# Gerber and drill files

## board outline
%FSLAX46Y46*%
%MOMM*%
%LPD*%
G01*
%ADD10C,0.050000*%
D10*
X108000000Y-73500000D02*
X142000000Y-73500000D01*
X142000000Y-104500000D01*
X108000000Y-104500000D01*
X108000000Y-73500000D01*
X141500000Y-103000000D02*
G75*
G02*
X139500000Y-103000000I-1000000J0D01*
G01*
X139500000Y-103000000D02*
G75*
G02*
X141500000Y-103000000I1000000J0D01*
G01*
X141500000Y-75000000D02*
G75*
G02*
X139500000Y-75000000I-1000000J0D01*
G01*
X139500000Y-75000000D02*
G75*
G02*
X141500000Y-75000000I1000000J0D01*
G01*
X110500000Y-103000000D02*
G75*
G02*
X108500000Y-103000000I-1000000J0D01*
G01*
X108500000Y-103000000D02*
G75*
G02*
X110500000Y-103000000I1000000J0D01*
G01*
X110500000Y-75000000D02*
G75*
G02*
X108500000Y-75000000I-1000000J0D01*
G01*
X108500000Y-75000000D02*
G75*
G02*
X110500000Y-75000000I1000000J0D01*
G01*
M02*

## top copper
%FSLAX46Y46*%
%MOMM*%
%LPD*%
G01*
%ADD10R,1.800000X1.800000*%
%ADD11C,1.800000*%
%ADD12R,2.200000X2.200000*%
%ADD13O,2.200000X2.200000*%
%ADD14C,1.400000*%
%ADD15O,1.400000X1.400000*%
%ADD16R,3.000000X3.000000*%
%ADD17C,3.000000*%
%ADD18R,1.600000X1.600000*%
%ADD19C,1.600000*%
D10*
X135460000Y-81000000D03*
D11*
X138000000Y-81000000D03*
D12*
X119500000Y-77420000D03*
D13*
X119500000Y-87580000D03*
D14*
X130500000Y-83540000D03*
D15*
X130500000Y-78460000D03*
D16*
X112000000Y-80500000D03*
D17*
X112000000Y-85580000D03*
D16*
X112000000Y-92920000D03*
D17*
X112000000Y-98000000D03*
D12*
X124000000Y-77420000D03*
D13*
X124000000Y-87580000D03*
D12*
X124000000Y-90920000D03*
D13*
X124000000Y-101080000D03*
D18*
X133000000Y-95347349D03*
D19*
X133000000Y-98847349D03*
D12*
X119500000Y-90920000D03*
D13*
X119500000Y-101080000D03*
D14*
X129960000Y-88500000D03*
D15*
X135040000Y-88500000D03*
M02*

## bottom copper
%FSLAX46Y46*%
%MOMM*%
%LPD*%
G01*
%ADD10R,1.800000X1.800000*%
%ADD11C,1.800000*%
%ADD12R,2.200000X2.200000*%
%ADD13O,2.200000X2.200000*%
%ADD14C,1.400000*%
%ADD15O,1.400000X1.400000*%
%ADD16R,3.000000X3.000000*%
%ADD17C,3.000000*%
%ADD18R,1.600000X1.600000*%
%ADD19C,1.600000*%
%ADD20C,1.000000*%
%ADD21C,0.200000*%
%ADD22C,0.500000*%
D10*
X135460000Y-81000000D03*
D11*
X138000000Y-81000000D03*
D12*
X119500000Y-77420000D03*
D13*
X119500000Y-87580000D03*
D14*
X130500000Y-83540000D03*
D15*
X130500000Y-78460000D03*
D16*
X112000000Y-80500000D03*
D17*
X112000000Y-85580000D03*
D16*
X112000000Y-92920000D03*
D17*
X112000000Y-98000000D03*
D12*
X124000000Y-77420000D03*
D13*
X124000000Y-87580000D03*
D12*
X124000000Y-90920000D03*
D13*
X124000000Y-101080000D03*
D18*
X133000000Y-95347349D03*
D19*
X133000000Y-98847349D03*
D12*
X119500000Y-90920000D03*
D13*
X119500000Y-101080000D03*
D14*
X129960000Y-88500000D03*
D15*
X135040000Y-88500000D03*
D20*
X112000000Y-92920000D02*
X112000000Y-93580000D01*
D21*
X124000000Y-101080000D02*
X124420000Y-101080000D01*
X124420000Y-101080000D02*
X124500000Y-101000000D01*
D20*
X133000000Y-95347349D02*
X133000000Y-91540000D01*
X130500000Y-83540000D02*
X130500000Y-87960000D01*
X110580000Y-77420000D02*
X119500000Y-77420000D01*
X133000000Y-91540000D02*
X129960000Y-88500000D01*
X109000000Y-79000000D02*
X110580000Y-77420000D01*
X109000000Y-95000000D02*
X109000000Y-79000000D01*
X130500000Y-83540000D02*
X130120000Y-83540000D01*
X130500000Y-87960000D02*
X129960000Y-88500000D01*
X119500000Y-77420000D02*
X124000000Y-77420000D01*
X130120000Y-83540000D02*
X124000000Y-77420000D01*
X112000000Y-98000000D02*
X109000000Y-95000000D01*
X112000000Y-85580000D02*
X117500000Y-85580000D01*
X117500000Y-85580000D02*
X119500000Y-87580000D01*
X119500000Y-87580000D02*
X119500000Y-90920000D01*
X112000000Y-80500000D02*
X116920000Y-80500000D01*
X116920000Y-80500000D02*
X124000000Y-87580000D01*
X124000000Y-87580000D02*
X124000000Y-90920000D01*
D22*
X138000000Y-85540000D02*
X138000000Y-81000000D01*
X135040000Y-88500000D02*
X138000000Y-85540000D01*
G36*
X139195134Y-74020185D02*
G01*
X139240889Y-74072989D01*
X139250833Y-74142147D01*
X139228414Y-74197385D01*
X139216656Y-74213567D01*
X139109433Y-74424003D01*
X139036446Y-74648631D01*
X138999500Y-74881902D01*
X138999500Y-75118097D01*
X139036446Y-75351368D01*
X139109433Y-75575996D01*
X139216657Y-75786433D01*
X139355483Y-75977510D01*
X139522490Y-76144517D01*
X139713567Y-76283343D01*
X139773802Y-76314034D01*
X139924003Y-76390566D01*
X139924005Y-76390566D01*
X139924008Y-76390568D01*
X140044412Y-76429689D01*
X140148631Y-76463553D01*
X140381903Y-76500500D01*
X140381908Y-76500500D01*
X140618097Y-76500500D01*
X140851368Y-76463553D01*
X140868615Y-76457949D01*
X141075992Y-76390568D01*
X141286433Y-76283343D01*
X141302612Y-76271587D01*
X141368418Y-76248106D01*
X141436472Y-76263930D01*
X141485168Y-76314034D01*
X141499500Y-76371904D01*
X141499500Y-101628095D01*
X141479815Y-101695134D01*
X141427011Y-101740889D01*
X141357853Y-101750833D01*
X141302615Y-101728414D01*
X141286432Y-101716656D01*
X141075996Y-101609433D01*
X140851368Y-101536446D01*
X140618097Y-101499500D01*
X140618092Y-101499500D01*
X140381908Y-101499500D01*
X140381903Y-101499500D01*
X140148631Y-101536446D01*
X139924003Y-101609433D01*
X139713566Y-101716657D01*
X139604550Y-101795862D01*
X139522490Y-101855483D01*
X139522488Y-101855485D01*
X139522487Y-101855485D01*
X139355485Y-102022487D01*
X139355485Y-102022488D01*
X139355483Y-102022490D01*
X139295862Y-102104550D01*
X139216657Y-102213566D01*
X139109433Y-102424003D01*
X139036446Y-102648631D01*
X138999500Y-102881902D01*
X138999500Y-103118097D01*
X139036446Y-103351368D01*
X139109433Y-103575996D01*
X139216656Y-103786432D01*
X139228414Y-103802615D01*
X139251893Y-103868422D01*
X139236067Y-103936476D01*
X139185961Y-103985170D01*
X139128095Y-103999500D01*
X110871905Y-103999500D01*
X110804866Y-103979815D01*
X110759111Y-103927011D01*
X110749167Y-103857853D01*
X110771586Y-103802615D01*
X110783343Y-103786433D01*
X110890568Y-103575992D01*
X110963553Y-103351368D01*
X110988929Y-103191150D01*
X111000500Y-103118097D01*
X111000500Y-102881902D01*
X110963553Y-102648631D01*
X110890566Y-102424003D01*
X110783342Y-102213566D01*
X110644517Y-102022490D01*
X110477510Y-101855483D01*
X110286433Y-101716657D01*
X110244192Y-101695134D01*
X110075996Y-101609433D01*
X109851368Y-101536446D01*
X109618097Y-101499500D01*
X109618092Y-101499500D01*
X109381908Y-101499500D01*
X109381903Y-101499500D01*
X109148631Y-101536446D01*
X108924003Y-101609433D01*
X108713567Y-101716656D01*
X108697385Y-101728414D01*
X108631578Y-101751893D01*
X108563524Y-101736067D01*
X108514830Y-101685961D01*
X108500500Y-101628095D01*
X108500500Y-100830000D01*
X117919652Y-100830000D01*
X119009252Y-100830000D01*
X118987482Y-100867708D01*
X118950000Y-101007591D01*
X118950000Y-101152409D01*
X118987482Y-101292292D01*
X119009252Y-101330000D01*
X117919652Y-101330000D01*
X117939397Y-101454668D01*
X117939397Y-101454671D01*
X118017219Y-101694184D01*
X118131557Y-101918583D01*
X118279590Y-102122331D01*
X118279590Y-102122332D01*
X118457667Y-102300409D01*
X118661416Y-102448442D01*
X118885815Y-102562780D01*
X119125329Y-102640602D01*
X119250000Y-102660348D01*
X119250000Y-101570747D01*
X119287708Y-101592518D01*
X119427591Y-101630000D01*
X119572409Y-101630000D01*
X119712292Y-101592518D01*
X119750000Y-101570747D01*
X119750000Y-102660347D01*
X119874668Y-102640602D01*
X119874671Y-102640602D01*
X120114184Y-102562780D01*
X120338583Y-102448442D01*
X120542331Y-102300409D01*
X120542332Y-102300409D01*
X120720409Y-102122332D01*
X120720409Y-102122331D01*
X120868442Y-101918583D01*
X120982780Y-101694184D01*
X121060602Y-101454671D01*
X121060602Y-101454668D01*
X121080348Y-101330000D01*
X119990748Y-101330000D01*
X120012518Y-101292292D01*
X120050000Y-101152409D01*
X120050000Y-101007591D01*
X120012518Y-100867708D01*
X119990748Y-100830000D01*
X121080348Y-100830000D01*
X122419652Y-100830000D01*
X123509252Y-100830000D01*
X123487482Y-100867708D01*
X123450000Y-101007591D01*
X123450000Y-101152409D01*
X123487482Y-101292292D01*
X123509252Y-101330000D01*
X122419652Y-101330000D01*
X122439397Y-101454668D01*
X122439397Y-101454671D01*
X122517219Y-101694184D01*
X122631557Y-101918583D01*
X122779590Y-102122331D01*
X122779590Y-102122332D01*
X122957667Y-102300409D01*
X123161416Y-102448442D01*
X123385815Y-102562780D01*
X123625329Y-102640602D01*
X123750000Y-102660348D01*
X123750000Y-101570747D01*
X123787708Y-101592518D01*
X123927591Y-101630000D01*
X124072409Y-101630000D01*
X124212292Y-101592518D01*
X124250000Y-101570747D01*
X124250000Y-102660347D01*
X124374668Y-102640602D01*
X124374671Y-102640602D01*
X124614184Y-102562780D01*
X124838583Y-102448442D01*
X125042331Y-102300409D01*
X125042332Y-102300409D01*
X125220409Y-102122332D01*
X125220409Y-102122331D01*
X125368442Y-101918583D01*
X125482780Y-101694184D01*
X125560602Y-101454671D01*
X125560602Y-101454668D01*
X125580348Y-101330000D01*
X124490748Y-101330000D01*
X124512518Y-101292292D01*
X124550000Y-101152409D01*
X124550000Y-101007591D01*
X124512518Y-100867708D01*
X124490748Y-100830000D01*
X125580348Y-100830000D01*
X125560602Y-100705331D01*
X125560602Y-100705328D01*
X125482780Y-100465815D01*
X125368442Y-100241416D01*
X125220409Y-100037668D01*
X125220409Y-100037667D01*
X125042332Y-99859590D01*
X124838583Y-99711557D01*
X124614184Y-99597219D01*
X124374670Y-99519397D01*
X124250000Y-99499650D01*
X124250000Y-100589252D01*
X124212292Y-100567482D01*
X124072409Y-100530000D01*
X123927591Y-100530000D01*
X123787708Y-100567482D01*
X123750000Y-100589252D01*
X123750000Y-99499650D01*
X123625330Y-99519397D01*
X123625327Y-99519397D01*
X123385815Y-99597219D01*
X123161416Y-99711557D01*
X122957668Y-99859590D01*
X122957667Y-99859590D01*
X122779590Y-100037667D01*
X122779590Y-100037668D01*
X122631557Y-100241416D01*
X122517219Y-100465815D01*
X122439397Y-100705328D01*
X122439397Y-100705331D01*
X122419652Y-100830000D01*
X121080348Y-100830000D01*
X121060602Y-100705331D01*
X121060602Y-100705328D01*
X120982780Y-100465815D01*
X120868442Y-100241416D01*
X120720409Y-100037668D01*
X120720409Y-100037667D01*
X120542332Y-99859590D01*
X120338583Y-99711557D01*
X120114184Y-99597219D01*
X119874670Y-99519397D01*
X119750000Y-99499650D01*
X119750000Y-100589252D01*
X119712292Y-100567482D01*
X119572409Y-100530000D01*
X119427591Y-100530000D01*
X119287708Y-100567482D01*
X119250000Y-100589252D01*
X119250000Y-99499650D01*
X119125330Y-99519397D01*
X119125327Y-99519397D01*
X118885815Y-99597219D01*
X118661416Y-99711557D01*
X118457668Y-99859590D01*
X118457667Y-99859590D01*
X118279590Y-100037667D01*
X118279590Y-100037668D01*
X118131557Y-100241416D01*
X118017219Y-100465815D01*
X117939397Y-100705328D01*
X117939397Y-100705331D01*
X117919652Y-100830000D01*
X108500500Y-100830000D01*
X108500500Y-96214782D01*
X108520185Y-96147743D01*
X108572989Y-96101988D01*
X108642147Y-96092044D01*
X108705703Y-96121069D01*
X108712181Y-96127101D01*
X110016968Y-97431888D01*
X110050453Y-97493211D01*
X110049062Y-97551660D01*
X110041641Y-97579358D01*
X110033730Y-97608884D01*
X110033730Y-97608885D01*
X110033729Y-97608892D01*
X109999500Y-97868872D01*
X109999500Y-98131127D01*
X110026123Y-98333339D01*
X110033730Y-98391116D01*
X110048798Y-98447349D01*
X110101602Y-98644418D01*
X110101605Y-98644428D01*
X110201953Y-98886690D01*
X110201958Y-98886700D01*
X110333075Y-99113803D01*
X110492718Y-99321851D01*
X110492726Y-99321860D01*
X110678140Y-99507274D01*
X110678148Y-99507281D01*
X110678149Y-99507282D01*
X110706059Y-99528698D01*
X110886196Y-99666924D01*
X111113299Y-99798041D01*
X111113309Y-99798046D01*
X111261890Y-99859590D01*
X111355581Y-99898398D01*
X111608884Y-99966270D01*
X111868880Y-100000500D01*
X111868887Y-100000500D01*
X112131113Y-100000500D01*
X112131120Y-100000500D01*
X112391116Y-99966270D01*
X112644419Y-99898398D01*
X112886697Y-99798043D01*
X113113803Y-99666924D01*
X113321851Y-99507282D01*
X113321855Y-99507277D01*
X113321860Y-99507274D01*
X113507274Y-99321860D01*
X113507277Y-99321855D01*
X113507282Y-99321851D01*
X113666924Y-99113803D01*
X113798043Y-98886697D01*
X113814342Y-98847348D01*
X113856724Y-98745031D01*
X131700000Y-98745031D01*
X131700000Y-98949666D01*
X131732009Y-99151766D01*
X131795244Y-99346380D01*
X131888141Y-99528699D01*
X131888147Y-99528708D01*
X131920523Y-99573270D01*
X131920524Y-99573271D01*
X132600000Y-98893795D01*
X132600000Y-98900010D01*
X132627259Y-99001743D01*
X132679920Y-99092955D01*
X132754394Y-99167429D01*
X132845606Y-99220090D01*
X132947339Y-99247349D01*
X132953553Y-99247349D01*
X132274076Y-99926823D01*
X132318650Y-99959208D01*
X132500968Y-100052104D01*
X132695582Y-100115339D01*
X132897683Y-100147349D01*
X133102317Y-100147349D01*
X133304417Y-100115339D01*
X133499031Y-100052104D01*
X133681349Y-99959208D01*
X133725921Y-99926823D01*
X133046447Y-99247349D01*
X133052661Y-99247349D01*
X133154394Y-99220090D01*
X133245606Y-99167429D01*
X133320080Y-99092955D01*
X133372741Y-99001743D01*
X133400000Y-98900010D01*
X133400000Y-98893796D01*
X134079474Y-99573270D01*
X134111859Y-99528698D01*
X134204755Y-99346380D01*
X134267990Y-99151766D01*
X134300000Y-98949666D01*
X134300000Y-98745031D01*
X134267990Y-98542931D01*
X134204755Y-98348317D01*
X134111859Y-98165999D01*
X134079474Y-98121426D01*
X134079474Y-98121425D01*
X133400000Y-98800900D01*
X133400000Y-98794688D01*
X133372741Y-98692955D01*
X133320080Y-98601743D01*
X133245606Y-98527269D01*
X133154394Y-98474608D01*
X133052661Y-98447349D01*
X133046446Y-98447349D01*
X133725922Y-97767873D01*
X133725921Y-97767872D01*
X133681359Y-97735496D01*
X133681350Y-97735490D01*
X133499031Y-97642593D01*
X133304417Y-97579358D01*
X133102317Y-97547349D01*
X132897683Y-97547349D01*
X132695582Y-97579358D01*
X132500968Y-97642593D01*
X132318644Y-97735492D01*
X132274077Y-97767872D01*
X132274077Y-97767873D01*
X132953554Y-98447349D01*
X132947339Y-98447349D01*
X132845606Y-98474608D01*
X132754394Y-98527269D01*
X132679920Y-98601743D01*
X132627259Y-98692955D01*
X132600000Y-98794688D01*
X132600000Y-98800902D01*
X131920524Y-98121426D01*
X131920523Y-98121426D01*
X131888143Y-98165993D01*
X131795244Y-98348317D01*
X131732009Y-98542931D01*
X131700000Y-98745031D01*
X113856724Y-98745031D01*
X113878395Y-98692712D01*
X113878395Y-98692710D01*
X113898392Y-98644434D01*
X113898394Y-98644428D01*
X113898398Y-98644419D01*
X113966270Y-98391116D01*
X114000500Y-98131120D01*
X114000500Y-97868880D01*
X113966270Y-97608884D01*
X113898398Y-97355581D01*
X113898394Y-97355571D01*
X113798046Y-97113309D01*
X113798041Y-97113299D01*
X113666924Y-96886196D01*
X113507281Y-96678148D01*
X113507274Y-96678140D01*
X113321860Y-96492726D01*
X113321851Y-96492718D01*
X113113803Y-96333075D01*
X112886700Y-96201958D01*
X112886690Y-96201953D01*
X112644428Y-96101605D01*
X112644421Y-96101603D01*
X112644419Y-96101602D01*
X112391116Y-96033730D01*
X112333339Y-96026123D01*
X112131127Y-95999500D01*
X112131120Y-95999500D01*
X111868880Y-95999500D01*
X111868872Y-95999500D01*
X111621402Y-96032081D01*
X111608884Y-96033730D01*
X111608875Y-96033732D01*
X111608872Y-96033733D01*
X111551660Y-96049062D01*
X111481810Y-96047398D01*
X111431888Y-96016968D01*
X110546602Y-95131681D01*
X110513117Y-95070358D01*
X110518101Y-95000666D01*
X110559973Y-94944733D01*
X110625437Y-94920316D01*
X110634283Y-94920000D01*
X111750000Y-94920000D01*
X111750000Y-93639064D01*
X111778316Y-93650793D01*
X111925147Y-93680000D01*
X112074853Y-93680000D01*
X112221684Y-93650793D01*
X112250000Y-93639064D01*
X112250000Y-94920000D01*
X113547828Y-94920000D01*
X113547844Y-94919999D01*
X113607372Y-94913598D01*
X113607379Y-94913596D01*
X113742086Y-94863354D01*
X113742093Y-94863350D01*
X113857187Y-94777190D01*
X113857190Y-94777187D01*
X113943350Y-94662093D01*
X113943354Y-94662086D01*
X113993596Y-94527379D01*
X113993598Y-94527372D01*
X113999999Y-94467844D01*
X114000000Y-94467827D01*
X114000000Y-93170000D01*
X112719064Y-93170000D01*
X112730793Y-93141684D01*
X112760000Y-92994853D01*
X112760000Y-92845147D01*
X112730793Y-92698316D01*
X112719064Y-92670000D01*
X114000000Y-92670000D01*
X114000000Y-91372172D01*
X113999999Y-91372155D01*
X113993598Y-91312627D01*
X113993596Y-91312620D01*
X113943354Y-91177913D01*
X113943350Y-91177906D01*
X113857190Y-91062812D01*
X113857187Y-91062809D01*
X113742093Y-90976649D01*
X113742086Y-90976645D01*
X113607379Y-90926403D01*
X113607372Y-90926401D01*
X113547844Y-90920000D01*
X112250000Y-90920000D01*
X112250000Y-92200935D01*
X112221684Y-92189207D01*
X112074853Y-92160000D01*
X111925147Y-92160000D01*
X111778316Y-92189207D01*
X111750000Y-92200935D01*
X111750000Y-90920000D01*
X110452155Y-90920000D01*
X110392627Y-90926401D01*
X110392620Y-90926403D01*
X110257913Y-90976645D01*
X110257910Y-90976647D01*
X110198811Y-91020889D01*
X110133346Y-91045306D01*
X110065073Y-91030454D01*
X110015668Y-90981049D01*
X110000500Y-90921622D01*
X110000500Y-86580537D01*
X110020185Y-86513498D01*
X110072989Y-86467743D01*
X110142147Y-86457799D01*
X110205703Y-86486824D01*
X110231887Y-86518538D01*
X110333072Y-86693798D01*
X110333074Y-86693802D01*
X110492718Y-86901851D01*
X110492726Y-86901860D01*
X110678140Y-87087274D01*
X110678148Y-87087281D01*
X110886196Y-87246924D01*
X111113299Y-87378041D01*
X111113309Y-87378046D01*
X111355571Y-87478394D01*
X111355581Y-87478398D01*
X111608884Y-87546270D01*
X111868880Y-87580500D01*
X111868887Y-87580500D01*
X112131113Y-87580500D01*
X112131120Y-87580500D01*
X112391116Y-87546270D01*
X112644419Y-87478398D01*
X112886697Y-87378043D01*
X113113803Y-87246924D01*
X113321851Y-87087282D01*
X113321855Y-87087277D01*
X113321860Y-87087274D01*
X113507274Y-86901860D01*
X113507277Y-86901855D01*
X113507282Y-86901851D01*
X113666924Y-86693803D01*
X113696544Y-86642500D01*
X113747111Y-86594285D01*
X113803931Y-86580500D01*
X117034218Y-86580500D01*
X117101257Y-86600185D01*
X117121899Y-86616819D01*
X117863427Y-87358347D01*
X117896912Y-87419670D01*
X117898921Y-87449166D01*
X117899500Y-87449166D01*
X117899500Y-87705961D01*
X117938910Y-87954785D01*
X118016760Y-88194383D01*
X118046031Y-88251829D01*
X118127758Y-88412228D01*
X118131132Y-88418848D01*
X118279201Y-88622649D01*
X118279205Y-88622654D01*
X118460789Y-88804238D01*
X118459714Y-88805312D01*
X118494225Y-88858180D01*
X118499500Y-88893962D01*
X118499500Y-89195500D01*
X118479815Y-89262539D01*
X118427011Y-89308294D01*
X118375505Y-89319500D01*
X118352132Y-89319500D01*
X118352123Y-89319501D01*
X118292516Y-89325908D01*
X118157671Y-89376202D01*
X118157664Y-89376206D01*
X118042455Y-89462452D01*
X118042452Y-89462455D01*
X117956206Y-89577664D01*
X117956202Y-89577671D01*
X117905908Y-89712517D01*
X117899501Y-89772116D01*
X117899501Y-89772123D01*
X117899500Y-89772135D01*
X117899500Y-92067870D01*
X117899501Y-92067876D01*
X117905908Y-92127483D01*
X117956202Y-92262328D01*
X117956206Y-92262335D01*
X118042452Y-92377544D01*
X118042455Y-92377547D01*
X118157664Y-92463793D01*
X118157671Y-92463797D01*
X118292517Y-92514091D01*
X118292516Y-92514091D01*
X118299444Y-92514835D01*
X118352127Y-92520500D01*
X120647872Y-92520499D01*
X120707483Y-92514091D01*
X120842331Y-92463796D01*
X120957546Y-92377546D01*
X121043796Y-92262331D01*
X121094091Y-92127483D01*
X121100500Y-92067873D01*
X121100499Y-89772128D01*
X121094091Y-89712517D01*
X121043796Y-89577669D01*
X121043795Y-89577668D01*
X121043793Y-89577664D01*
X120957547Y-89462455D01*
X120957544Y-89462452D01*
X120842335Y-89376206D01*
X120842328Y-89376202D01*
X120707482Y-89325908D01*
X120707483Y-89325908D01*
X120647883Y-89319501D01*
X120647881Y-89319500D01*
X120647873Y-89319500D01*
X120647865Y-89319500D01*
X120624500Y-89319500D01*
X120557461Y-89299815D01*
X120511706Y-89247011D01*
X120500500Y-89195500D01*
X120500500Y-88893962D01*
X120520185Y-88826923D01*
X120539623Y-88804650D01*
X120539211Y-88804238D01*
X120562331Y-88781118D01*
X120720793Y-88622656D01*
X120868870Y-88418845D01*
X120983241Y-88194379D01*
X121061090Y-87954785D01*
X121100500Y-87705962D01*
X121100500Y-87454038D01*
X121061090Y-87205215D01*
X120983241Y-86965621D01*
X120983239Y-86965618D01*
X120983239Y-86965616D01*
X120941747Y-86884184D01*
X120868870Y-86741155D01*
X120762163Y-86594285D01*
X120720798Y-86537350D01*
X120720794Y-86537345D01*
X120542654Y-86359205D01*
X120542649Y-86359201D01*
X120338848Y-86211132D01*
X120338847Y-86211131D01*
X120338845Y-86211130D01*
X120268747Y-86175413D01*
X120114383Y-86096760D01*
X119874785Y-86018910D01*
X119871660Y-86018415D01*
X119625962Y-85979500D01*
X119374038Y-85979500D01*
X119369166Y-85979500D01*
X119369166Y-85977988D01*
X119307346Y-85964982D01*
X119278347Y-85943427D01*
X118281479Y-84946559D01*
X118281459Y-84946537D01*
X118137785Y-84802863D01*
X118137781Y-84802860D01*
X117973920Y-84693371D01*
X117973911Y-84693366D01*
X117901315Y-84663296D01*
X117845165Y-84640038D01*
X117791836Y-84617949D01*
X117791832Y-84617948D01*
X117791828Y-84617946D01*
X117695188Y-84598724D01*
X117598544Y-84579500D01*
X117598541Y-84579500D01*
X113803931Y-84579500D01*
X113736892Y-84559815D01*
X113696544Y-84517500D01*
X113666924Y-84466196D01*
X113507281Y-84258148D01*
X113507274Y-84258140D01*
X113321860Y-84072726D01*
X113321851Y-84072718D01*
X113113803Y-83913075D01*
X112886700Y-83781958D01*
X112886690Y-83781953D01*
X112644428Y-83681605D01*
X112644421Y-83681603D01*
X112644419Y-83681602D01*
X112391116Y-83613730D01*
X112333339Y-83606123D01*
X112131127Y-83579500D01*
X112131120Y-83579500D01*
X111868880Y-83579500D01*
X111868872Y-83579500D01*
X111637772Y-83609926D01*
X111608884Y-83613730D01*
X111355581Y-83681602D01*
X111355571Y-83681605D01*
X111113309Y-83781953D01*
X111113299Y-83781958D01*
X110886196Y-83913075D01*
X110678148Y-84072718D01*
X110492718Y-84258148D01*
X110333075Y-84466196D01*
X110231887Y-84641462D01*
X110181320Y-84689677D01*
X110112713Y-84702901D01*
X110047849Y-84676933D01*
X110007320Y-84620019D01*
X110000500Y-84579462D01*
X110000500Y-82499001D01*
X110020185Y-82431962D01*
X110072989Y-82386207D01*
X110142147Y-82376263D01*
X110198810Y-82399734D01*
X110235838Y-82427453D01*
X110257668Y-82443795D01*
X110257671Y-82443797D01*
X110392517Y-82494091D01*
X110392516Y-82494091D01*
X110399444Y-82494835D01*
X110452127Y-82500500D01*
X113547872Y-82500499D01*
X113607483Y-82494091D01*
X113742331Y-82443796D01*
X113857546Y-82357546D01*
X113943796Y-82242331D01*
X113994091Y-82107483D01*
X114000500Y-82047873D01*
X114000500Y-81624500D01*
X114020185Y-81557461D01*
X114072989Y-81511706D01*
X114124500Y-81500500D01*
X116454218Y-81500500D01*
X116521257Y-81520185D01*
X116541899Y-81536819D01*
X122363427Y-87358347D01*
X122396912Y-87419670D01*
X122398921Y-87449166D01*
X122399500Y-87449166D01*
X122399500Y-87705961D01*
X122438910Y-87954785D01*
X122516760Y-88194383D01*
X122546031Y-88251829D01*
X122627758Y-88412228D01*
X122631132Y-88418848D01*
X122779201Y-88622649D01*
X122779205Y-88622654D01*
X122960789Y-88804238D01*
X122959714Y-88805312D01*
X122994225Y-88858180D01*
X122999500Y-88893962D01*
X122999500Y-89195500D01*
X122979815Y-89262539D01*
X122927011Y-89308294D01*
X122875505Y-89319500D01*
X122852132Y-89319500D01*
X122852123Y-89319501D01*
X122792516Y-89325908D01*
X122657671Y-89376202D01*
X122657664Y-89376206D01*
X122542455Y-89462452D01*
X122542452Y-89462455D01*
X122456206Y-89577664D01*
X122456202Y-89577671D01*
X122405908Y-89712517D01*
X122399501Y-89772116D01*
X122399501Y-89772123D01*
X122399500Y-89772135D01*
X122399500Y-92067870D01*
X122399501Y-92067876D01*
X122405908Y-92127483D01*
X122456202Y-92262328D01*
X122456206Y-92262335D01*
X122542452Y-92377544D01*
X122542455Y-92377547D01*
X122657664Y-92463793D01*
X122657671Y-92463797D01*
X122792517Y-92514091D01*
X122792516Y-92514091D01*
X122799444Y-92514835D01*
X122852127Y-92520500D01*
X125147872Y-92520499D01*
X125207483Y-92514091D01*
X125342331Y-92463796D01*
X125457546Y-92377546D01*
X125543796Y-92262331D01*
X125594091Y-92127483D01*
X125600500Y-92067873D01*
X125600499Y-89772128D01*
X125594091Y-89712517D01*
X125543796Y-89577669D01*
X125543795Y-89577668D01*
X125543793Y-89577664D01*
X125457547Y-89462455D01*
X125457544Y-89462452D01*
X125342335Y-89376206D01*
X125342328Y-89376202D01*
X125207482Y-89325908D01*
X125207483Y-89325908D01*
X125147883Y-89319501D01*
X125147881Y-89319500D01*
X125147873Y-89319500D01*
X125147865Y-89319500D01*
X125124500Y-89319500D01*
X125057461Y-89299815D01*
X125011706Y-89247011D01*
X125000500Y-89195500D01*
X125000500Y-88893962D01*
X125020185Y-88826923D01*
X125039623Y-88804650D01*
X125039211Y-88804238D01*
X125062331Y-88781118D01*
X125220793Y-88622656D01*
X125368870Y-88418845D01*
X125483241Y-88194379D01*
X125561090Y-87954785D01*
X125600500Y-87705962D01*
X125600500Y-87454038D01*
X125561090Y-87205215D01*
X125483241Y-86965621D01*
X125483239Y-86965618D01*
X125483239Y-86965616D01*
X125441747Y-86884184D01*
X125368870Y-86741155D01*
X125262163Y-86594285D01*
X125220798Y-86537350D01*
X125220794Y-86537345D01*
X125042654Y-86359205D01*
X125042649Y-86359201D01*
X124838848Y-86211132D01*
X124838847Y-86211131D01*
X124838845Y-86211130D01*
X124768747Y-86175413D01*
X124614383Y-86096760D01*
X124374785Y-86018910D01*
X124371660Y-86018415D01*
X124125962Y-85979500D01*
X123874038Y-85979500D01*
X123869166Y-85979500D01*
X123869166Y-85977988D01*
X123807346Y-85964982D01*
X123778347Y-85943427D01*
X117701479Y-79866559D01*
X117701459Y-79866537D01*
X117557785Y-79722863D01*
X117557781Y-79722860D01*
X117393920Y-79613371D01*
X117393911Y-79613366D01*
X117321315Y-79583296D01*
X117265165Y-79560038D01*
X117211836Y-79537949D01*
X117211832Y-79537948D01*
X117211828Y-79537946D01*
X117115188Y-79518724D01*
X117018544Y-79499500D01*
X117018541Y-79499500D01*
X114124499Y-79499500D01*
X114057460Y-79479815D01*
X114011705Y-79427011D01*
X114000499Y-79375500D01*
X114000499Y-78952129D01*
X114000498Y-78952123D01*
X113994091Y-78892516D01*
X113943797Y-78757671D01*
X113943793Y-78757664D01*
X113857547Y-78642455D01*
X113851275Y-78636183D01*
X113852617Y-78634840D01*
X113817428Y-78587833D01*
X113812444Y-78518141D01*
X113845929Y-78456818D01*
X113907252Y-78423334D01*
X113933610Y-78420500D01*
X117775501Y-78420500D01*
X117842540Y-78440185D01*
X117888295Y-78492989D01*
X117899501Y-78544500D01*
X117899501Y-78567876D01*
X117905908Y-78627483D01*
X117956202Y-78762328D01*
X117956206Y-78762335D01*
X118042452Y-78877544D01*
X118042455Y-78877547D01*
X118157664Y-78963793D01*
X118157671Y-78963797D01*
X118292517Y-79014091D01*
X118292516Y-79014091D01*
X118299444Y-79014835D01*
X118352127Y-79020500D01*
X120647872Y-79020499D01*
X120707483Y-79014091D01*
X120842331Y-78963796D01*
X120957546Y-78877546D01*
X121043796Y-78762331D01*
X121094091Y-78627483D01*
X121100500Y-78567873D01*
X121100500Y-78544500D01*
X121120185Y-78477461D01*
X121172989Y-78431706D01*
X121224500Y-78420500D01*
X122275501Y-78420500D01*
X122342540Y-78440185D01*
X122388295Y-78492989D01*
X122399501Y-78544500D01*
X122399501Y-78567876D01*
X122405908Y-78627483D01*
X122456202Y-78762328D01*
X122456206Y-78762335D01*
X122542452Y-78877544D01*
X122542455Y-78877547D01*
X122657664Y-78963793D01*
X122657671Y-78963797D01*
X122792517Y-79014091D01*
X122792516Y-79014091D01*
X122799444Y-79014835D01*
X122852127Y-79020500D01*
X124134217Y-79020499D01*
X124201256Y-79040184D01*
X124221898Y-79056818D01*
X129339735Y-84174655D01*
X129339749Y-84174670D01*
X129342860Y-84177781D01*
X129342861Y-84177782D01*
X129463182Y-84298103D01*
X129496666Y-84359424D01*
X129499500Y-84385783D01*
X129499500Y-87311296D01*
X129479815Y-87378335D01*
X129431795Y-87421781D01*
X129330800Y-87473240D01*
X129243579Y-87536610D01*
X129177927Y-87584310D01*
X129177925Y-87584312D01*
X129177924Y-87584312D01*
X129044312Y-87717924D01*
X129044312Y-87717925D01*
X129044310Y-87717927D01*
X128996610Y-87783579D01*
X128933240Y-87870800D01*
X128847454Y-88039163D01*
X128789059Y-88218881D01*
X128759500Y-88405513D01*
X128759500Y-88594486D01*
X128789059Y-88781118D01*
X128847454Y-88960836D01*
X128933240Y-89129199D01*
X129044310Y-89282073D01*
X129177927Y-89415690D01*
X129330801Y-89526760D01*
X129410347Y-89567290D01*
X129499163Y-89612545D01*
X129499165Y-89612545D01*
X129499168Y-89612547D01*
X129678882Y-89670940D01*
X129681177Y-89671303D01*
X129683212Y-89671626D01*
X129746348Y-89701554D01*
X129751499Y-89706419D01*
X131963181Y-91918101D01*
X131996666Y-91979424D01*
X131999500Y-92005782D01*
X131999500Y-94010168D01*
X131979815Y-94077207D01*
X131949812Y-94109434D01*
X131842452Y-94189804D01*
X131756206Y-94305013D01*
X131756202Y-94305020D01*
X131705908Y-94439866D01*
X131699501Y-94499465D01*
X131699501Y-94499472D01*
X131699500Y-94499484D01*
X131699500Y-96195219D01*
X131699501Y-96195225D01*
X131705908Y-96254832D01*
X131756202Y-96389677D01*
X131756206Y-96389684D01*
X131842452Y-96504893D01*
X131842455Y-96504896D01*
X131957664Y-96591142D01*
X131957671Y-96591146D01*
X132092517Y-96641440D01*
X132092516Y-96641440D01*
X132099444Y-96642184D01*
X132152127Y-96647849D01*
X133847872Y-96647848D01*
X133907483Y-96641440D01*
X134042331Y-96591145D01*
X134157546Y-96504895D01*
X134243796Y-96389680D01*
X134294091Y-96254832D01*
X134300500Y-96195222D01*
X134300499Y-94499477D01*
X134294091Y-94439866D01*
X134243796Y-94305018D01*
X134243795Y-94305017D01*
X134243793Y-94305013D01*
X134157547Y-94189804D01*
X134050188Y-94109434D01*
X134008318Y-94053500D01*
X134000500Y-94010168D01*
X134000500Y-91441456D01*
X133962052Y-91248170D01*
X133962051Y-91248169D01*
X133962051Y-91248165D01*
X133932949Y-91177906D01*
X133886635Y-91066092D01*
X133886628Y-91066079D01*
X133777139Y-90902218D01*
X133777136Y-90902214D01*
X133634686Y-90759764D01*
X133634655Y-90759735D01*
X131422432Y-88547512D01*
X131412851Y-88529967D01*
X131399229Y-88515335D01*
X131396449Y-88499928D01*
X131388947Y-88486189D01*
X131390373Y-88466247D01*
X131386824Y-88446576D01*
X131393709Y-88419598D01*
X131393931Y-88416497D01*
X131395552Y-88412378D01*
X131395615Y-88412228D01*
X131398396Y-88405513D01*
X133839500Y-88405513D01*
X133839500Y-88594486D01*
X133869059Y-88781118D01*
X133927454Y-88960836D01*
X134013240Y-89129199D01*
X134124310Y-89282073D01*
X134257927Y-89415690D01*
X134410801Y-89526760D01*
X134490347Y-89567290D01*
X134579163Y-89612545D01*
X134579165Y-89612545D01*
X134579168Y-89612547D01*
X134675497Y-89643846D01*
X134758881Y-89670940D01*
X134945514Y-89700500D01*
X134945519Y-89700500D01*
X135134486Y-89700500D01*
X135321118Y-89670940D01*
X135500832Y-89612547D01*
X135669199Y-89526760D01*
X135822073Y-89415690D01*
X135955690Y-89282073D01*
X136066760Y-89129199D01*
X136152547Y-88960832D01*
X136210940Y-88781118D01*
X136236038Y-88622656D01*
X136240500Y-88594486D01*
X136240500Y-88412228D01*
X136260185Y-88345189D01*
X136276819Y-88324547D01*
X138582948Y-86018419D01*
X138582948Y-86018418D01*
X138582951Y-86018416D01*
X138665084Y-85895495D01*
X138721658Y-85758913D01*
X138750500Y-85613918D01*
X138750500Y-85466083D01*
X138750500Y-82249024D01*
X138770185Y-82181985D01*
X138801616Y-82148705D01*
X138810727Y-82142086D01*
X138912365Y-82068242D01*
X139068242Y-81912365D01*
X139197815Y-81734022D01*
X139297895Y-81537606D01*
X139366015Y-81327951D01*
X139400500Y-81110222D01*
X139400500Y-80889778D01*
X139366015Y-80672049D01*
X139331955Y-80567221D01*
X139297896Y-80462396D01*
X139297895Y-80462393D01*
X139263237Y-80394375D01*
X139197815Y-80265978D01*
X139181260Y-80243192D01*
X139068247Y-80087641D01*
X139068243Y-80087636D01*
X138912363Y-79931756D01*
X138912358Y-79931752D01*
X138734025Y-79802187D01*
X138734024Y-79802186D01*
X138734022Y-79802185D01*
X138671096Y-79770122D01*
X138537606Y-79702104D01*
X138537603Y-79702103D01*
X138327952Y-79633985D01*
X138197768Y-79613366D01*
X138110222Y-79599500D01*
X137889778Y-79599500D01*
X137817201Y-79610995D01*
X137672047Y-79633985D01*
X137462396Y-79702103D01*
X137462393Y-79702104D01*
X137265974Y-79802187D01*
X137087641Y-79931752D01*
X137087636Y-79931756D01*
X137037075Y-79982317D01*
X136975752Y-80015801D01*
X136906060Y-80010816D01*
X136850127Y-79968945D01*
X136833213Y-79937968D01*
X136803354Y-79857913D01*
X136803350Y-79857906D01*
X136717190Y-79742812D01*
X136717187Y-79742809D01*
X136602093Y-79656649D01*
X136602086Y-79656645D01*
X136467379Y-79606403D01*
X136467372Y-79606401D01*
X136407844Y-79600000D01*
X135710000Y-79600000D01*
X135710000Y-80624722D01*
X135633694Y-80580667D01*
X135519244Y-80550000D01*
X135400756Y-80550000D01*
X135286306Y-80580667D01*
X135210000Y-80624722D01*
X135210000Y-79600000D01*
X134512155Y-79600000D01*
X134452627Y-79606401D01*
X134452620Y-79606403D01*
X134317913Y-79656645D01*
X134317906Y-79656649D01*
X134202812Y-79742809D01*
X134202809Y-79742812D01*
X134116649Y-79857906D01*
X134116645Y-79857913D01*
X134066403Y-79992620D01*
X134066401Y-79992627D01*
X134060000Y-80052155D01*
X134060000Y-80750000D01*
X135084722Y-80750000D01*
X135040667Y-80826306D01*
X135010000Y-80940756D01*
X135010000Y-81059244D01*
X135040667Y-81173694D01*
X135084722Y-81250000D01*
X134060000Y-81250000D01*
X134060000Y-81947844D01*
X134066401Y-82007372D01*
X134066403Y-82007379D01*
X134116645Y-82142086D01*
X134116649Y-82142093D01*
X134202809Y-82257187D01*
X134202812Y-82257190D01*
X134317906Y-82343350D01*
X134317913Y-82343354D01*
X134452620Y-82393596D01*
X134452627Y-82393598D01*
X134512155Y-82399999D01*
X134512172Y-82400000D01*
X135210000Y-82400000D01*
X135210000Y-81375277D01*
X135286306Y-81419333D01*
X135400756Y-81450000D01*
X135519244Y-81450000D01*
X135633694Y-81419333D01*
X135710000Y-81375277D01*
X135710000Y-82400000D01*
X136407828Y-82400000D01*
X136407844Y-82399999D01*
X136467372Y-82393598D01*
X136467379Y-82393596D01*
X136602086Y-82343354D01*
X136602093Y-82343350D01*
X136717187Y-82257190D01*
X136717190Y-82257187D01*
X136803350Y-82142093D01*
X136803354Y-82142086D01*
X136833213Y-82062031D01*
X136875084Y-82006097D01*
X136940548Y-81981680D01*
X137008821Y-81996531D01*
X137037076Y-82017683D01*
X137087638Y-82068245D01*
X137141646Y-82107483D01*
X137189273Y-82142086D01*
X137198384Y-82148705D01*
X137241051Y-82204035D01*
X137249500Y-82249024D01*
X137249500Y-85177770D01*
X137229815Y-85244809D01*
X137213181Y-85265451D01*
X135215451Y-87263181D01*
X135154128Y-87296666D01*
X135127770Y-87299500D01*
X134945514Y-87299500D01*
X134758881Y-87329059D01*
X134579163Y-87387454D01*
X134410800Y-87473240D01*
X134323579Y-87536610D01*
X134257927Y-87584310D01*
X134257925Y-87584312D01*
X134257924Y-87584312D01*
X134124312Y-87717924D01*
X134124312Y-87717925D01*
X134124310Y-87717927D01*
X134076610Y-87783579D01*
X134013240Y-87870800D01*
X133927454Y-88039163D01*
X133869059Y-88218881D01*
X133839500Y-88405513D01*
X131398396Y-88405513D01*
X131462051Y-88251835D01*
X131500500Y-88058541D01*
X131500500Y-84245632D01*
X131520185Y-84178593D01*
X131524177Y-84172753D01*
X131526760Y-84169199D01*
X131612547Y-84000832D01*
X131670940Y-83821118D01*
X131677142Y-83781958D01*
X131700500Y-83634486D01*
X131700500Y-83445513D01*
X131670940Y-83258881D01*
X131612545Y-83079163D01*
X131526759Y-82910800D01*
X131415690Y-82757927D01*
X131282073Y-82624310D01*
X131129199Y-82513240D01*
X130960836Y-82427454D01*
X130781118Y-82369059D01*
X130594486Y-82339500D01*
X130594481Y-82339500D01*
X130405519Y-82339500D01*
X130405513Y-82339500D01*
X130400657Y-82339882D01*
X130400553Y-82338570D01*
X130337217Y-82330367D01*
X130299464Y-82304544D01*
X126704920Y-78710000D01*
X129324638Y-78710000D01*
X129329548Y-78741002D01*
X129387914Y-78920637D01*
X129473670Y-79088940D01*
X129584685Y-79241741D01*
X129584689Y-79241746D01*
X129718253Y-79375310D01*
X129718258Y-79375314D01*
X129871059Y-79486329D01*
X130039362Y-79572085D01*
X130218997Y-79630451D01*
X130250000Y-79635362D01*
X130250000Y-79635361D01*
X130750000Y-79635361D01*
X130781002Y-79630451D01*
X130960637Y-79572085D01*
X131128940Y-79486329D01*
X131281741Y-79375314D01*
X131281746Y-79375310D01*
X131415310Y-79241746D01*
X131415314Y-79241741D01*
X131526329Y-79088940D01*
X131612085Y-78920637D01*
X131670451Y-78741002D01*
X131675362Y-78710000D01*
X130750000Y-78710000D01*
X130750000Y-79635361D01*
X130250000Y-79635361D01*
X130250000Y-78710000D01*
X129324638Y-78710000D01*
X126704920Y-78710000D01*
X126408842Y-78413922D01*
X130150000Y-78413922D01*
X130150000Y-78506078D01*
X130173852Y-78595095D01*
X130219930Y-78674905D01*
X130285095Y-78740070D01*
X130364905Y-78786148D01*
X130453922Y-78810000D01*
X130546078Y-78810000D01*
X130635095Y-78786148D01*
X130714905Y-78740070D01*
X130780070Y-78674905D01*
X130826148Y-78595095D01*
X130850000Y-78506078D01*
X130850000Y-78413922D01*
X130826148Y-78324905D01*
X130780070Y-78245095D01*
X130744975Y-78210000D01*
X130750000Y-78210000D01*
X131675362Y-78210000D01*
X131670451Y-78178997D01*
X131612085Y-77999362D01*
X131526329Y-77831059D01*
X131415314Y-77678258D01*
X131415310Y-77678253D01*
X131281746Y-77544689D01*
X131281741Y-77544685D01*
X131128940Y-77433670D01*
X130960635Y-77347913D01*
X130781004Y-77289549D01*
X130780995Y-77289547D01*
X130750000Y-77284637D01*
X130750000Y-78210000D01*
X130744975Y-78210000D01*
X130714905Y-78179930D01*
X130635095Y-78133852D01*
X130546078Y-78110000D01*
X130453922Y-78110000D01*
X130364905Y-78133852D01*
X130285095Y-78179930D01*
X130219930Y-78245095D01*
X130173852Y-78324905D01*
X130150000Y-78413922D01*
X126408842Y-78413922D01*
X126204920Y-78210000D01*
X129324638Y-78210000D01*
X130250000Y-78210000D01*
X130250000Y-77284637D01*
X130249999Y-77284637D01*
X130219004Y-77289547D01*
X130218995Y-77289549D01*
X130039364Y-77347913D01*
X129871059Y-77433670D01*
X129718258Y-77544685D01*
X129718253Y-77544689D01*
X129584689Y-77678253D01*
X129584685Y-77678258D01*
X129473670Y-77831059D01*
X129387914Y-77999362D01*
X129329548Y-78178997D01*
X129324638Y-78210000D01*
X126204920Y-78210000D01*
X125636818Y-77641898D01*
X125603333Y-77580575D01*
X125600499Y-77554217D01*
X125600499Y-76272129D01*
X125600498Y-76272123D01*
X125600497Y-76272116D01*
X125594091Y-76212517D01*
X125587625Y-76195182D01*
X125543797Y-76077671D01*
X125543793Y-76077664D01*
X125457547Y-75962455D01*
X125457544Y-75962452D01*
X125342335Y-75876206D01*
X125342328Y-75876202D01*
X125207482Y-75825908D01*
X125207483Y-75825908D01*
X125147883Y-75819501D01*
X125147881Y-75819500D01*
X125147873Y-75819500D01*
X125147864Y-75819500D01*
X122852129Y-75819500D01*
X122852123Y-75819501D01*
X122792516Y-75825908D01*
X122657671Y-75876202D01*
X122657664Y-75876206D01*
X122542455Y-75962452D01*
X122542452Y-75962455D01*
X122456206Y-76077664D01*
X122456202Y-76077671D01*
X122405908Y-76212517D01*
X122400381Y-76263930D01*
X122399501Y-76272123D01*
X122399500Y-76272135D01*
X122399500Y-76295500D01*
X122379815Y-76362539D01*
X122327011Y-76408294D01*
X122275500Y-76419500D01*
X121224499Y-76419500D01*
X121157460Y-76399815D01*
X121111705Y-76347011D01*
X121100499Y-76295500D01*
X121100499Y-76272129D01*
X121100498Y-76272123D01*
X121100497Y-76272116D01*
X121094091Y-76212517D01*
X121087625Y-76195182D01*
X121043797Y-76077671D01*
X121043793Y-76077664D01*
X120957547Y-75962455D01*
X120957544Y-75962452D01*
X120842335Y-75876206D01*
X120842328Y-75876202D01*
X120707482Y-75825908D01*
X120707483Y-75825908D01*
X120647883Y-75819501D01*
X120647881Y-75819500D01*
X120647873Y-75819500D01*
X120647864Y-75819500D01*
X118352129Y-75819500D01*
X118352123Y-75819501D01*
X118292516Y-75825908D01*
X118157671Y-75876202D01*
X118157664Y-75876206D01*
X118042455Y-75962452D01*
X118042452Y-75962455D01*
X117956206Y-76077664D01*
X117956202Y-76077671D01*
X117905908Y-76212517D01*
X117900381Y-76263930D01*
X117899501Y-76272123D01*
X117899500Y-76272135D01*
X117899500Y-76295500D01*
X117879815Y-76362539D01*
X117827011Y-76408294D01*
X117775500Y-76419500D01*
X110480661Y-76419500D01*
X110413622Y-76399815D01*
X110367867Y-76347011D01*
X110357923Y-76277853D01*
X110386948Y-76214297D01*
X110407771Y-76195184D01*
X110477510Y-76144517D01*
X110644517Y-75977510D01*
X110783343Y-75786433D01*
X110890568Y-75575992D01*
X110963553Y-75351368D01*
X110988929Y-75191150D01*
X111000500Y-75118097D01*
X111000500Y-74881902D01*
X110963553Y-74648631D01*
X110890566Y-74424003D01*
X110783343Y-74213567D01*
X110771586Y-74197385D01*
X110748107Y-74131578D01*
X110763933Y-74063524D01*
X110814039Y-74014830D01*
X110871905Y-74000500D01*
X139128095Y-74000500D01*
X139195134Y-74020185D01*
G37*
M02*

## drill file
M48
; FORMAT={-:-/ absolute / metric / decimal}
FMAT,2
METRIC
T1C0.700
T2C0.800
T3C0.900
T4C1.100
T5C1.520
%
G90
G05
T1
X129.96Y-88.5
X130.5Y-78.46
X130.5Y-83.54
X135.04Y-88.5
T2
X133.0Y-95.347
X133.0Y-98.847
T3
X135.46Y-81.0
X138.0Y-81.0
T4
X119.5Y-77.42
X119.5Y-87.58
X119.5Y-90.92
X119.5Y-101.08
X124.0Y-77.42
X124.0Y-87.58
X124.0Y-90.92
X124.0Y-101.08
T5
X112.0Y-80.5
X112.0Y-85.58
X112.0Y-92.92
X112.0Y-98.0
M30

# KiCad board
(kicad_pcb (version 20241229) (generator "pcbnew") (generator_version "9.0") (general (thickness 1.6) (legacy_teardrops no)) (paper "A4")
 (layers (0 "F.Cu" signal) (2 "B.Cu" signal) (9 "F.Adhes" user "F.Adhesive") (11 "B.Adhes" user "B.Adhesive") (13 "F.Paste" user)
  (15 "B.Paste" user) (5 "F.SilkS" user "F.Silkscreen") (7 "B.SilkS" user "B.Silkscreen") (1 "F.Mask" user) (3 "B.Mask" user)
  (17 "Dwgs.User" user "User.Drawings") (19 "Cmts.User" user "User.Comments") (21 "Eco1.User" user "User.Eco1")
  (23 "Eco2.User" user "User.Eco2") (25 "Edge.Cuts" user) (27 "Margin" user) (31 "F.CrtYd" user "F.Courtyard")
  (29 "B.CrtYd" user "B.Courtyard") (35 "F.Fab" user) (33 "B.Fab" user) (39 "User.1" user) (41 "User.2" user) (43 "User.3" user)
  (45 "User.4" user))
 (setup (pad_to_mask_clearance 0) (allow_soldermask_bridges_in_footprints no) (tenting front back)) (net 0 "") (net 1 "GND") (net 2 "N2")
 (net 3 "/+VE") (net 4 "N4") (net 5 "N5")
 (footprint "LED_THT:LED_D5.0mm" (layer "F.Cu") (at 135.46 81)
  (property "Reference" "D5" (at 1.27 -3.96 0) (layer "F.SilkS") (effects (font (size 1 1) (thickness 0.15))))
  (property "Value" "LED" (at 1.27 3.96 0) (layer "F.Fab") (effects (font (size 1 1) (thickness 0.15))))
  (pad "1" thru_hole rect (at 0 0) (size 1.8 1.8) (drill 0.9) (layers "*.Cu" "*.Mask") (remove_unused_layers no) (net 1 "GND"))
  (pad "2" thru_hole circle (at 2.54 0) (size 1.8 1.8) (drill 0.9) (layers "*.Cu" "*.Mask") (remove_unused_layers no) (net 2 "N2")))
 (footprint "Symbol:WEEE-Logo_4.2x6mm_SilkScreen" (layer "F.Cu") (at 138.5 91)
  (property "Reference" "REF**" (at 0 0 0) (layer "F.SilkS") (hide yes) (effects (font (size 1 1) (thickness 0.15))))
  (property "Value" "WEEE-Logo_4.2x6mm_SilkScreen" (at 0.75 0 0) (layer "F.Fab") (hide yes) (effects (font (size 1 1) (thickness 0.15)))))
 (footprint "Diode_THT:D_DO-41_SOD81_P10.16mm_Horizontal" (layer "F.Cu") (at 119.5 77.42 -90)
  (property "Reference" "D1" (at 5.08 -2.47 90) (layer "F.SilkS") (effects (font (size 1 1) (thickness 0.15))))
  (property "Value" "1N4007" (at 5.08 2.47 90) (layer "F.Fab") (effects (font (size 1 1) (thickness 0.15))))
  (pad "1" thru_hole rect (at 0 0 270) (size 2.2 2.2) (drill 1.1) (layers "*.Cu" "*.Mask") (remove_unused_layers no) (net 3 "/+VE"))
  (pad "2" thru_hole oval (at 10.16 0 270) (size 2.2 2.2) (drill 1.1) (layers "*.Cu" "*.Mask") (remove_unused_layers no) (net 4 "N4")))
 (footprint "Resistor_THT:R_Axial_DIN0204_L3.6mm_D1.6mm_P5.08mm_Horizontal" (layer "F.Cu") (at 130.5 83.54 90)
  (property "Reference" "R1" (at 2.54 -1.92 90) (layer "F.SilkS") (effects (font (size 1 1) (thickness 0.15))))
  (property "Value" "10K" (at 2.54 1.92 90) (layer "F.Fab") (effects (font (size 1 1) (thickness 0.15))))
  (pad "1" thru_hole circle (at 0 0 90) (size 1.4 1.4) (drill 0.7) (layers "*.Cu" "*.Mask") (remove_unused_layers no) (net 3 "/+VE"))
  (pad "2" thru_hole oval (at 5.08 0 90) (size 1.4 1.4) (drill 0.7) (layers "*.Cu" "*.Mask") (remove_unused_layers no) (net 1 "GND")))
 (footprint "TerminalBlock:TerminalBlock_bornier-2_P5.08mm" (layer "F.Cu") (at 112 80.5 -90)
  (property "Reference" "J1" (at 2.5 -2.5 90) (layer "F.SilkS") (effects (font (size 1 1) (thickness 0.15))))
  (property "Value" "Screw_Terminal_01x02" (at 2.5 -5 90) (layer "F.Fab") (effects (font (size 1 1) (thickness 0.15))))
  (pad "1" thru_hole rect (at 0 0 270) (size 3 3) (drill 1.52) (layers "*.Cu" "*.Mask") (remove_unused_layers no) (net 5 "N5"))
  (pad "2" thru_hole circle (at 5.08 0 270) (size 3 3) (drill 1.52) (layers "*.Cu" "*.Mask") (remove_unused_layers no) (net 4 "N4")))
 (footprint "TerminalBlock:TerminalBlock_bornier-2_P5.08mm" (layer "F.Cu") (at 112 92.92 -90)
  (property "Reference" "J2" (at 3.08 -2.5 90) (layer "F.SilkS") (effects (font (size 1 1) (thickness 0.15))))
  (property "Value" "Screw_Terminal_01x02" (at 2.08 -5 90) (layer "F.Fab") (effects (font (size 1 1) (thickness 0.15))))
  (pad "1" thru_hole rect (at 0 0 270) (size 3 3) (drill 1.52) (layers "*.Cu" "*.Mask") (remove_unused_layers no) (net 1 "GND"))
  (pad "2" thru_hole circle (at 5.08 0 270) (size 3 3) (drill 1.52) (layers "*.Cu" "*.Mask") (remove_unused_layers no) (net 3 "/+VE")))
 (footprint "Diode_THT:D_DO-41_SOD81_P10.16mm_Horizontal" (layer "F.Cu") (at 124 77.42 -90)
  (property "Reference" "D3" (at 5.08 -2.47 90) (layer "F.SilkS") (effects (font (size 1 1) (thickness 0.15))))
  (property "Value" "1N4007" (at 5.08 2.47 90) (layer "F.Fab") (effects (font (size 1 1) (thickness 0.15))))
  (pad "1" thru_hole rect (at 0 0 270) (size 2.2 2.2) (drill 1.1) (layers "*.Cu" "*.Mask") (remove_unused_layers no) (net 3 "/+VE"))
  (pad "2" thru_hole oval (at 10.16 0 270) (size 2.2 2.2) (drill 1.1) (layers "*.Cu" "*.Mask") (remove_unused_layers no) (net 5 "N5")))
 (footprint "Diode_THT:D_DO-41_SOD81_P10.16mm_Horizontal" (layer "F.Cu") (at 124 90.92 -90)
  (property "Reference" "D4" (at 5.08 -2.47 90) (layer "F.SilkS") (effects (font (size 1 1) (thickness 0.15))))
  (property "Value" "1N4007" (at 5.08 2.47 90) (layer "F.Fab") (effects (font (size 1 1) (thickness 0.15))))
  (pad "1" thru_hole rect (at 0 0 270) (size 2.2 2.2) (drill 1.1) (layers "*.Cu" "*.Mask") (remove_unused_layers no) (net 5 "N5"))
  (pad "2" thru_hole oval (at 10.16 0 270) (size 2.2 2.2) (drill 1.1) (layers "*.Cu" "*.Mask") (remove_unused_layers no) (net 1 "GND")))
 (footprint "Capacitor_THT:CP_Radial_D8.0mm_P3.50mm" (layer "F.Cu") (at 133 95.347349 -90)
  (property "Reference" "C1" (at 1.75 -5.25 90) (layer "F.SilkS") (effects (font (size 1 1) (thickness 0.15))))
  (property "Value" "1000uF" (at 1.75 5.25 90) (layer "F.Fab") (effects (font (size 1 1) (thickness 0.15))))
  (pad "1" thru_hole rect (at 0 0 270) (size 1.6 1.6) (drill 0.8) (layers "*.Cu" "*.Mask") (remove_unused_layers no) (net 3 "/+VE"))
  (pad "2" thru_hole circle (at 3.5 0 270) (size 1.6 1.6) (drill 0.8) (layers "*.Cu" "*.Mask") (remove_unused_layers no) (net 1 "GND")))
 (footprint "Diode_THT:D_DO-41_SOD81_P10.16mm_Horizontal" (layer "F.Cu") (at 119.5 90.92 -90)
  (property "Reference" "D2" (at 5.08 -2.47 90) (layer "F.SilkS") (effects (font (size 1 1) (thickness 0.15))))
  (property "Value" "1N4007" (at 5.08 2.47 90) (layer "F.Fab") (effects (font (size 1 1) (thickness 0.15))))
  (pad "1" thru_hole rect (at 0 0 270) (size 2.2 2.2) (drill 1.1) (layers "*.Cu" "*.Mask") (remove_unused_layers no) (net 4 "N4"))
  (pad "2" thru_hole oval (at 10.16 0 270) (size 2.2 2.2) (drill 1.1) (layers "*.Cu" "*.Mask") (remove_unused_layers no) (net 1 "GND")))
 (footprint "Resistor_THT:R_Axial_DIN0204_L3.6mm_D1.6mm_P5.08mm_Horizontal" (layer "F.Cu") (at 129.96 88.5)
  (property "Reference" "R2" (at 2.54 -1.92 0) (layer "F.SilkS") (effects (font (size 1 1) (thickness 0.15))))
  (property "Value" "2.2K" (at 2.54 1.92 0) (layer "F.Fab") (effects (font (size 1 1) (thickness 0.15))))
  (pad "1" thru_hole circle (at 0 0) (size 1.4 1.4) (drill 0.7) (layers "*.Cu" "*.Mask") (remove_unused_layers no) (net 3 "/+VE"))
  (pad "2" thru_hole oval (at 5.08 0) (size 1.4 1.4) (drill 0.7) (layers "*.Cu" "*.Mask") (remove_unused_layers no) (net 2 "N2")))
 (gr_rect (start 108 73.5) (end 142 104.5) (stroke (width 0.05) (type default)) (fill no) (layer "Edge.Cuts"))
 (gr_circle (center 140.5 103) (end 141.5 103) (stroke (width 0.05) (type default)) (fill no) (layer "Edge.Cuts"))
 (gr_circle (center 140.5 75) (end 141.5 75) (stroke (width 0.05) (type default)) (fill no) (layer "Edge.Cuts"))
 (gr_circle (center 109.5 103) (end 110.5 103) (stroke (width 0.05) (type default)) (fill no) (layer "Edge.Cuts"))
 (gr_circle (center 109.5 75) (end 110.5 75) (stroke (width 0.05) (type default)) (fill no) (layer "Edge.Cuts"))
 (segment (start 112 92.92) (end 112 93.58) (width 1) (layer "B.Cu") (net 1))
 (segment (start 124 101.08) (end 124.42 101.08) (width 0.2) (layer "B.Cu") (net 1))
 (segment (start 124.42 101.08) (end 124.5 101) (width 0.2) (layer "B.Cu") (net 1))
 (segment (start 133 95.347349) (end 133 91.54) (width 1) (layer "B.Cu") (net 3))
 (segment (start 130.5 83.54) (end 130.5 87.96) (width 1) (layer "B.Cu") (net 3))
 (segment (start 110.58 77.42) (end 119.5 77.42) (width 1) (layer "B.Cu") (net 3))
 (segment (start 133 91.54) (end 129.96 88.5) (width 1) (layer "B.Cu") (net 3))
 (segment (start 109 79) (end 110.58 77.42) (width 1) (layer "B.Cu") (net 3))
 (segment (start 109 95) (end 109 79) (width 1) (layer "B.Cu") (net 3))
 (segment (start 130.5 83.54) (end 130.12 83.54) (width 1) (layer "B.Cu") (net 3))
 (segment (start 130.5 87.96) (end 129.96 88.5) (width 1) (layer "B.Cu") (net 3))
 (segment (start 119.5 77.42) (end 124 77.42) (width 1) (layer "B.Cu") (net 3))
 (segment (start 130.12 83.54) (end 124 77.42) (width 1) (layer "B.Cu") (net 3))
 (segment (start 112 98) (end 109 95) (width 1) (layer "B.Cu") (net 3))
 (segment (start 112 85.58) (end 117.5 85.58) (width 1) (layer "B.Cu") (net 4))
 (segment (start 117.5 85.58) (end 119.5 87.58) (width 1) (layer "B.Cu") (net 4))
 (segment (start 119.5 87.58) (end 119.5 90.92) (width 1) (layer "B.Cu") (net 4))
 (segment (start 112 80.5) (end 116.92 80.5) (width 1) (layer "B.Cu") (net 5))
 (segment (start 116.92 80.5) (end 124 87.58) (width 1) (layer "B.Cu") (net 5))
 (segment (start 124 87.58) (end 124 90.92) (width 1) (layer "B.Cu") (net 5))
 (segment (start 138 85.54) (end 138 81) (width 0.5) (layer "B.Cu") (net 2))
 (segment (start 135.04 88.5) (end 138 85.54) (width 0.5) (layer "B.Cu") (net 2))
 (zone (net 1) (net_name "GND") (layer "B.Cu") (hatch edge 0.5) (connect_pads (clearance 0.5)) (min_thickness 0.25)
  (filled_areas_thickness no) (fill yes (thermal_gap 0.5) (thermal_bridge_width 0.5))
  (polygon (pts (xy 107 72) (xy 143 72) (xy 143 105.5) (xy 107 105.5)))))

